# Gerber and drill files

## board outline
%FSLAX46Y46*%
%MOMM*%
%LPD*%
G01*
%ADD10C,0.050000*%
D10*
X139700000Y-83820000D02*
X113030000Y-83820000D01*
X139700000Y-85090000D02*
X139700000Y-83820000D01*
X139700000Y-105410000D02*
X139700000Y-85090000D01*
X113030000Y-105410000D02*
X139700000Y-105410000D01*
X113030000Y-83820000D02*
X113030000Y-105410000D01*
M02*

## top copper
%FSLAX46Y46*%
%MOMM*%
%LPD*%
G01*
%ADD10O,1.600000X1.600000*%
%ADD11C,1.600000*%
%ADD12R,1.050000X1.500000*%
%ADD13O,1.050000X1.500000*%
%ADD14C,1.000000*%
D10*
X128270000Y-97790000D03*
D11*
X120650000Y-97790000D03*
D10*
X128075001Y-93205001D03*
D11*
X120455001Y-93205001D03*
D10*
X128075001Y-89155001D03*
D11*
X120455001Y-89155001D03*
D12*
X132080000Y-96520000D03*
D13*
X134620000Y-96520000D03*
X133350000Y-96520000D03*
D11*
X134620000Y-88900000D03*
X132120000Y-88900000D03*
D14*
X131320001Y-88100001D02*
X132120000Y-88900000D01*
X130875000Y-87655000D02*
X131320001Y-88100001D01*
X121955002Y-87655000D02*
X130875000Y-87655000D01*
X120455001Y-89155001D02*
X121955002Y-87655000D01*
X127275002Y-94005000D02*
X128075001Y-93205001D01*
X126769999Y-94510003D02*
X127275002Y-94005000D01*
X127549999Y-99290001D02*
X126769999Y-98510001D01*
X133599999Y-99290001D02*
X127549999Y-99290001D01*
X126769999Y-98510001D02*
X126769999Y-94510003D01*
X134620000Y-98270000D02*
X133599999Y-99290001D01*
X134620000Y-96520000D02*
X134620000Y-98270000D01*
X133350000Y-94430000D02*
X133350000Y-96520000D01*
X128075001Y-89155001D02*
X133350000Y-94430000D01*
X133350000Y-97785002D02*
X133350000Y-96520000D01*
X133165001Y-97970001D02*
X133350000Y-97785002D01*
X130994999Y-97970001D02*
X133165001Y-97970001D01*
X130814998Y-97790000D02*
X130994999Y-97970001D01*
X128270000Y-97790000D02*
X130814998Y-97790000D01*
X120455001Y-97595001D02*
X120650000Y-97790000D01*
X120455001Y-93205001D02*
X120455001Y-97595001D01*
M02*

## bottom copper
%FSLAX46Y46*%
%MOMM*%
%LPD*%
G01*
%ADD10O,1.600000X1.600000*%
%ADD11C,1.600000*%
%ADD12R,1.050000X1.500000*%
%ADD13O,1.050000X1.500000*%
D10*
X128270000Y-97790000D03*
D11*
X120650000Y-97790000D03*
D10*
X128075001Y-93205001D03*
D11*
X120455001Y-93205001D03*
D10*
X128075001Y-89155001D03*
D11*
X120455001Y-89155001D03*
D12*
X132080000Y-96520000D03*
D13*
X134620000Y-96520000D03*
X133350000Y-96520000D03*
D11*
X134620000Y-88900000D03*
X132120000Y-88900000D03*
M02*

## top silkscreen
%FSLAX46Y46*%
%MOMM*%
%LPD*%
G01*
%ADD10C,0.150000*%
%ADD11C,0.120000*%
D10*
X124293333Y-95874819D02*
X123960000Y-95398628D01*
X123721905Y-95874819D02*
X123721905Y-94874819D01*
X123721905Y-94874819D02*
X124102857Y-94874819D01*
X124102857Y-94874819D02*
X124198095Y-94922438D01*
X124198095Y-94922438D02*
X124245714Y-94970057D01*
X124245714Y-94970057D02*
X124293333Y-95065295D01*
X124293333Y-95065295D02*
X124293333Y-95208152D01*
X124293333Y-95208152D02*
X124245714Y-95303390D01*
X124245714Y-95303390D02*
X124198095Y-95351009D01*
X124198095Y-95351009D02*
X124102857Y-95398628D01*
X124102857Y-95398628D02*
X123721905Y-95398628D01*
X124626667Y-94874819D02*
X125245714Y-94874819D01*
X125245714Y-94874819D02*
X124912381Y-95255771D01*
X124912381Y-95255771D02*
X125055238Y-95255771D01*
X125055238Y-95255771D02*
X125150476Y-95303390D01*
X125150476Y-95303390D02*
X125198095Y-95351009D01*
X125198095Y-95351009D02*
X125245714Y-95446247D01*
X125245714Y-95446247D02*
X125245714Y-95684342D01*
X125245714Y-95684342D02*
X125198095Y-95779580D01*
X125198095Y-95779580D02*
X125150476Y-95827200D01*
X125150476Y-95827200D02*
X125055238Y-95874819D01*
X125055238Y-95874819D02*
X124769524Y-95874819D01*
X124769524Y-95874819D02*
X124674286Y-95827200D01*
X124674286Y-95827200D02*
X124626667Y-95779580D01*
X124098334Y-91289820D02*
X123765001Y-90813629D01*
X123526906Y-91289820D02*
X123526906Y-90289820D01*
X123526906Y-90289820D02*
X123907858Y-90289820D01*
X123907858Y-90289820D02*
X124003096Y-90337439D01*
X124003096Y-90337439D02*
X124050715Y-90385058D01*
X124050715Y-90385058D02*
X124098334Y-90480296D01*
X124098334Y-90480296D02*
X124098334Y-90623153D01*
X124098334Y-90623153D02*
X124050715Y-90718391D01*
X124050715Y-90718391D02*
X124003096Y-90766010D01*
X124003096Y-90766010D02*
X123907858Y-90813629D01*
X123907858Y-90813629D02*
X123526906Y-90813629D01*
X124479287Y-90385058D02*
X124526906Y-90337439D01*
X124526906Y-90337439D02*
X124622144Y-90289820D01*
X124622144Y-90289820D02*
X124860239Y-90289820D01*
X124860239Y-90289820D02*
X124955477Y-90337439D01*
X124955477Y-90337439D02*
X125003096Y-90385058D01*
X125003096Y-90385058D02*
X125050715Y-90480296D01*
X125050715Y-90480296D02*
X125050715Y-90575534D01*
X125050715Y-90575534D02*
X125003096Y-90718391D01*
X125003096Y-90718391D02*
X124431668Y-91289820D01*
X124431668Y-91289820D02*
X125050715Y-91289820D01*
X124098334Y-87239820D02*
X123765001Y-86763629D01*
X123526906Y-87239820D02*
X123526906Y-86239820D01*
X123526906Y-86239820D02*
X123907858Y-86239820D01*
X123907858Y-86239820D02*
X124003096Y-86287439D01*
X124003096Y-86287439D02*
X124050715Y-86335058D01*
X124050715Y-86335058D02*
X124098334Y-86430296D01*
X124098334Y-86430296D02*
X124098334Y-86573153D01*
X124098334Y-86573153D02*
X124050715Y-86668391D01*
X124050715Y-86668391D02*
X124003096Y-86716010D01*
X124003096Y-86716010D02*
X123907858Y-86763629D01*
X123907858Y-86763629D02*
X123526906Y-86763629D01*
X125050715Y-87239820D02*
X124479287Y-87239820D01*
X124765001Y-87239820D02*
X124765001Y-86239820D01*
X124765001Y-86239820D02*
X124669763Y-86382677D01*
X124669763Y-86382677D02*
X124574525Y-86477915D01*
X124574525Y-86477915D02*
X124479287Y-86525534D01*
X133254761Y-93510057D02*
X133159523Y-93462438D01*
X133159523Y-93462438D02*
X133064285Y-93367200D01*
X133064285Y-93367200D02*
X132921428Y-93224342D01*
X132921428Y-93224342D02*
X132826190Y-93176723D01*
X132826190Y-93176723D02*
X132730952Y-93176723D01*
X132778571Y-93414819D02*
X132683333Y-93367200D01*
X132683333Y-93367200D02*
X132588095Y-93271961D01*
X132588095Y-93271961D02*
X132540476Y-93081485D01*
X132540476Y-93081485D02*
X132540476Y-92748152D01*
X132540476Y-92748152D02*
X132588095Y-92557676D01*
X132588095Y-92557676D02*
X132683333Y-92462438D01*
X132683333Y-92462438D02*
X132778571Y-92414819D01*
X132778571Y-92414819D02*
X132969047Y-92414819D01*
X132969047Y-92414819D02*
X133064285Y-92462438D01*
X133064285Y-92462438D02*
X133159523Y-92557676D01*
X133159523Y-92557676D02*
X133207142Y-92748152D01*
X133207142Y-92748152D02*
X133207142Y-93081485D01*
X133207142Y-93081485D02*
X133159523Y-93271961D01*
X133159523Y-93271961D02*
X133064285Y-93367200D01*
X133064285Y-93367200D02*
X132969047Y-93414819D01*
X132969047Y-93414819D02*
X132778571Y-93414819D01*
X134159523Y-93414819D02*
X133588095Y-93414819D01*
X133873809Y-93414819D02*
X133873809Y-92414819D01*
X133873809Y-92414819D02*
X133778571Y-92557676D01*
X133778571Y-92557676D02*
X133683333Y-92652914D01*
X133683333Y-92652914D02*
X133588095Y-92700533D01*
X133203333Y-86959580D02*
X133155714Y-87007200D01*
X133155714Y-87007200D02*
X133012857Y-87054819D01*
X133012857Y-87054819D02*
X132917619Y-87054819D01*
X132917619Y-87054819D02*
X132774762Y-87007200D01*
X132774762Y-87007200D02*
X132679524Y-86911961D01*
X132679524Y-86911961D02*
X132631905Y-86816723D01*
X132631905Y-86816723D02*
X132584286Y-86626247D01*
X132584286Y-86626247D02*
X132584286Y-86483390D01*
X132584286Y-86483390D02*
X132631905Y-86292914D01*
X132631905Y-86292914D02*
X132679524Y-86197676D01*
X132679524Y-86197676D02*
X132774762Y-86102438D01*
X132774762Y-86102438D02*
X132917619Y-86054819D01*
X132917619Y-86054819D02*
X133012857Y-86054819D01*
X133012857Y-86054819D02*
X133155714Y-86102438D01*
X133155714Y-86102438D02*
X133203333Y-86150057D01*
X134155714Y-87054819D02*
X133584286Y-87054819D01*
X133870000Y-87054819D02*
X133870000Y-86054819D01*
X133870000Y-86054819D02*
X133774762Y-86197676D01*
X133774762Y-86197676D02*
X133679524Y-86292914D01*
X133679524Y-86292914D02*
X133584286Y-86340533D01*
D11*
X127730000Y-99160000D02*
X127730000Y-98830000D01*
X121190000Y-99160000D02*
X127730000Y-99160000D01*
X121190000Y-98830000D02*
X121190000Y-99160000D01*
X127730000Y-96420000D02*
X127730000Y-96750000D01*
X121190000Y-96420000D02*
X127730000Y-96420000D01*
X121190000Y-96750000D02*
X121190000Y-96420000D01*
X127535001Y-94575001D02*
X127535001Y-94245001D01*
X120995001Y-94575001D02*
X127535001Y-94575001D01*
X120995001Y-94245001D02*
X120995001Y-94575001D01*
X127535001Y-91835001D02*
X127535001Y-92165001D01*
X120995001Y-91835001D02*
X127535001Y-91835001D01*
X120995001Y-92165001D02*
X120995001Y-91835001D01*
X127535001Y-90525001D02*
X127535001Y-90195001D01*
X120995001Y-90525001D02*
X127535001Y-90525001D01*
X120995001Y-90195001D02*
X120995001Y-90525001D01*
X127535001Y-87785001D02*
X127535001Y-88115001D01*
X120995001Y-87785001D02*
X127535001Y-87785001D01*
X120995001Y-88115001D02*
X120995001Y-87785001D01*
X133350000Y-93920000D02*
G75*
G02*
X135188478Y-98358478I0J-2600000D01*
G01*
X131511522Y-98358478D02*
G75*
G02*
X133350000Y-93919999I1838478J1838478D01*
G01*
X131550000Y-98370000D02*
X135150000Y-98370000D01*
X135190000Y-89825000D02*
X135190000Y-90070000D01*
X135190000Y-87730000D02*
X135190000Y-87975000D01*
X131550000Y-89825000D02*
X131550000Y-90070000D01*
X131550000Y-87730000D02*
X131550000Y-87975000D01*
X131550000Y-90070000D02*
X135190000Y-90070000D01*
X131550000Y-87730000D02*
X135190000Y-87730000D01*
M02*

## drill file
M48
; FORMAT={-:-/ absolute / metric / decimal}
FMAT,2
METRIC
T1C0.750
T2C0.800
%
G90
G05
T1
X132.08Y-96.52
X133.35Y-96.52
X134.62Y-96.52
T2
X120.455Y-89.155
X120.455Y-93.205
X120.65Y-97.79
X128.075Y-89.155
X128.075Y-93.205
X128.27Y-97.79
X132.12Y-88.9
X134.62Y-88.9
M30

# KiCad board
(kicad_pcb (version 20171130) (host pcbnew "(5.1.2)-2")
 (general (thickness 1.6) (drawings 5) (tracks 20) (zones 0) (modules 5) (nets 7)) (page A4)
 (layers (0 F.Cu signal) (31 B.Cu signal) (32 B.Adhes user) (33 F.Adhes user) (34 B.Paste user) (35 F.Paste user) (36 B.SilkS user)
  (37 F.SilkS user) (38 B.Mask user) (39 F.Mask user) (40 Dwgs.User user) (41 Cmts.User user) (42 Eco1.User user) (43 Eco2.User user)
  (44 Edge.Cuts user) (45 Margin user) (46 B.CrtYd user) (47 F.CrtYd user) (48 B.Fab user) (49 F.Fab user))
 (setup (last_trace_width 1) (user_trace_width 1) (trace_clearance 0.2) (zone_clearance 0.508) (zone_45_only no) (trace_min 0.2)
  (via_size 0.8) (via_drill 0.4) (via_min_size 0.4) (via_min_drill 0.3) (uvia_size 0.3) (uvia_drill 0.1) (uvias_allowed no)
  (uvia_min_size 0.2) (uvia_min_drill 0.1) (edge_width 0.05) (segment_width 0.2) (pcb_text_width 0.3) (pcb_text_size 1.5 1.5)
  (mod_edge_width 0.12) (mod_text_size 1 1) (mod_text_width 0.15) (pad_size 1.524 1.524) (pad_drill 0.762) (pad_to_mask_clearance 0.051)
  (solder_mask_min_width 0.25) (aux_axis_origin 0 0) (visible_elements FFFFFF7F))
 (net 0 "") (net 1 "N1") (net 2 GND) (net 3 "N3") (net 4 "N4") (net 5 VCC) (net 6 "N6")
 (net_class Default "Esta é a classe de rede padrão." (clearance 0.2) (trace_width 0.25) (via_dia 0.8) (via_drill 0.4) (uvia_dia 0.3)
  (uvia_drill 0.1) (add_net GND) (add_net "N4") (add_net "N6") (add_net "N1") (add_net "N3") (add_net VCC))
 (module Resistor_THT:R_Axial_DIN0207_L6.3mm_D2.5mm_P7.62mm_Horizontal (layer F.Cu) (at 120.65 97.79)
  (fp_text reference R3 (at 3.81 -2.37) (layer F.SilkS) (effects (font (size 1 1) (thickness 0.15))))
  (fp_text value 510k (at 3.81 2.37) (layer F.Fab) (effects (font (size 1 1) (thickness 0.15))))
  (fp_line (start 7.08 1.37) (end 7.08 1.04) (layer F.SilkS) (width 0.12))
  (fp_line (start 0.54 1.37) (end 7.08 1.37) (layer F.SilkS) (width 0.12))
  (fp_line (start 0.54 1.04) (end 0.54 1.37) (layer F.SilkS) (width 0.12))
  (fp_line (start 7.08 -1.37) (end 7.08 -1.04) (layer F.SilkS) (width 0.12))
  (fp_line (start 0.54 -1.37) (end 7.08 -1.37) (layer F.SilkS) (width 0.12))
  (fp_line (start 0.54 -1.04) (end 0.54 -1.37) (layer F.SilkS) (width 0.12))
  (pad 2 thru_hole oval (at 7.62 0) (size 1.6 1.6) (drill 0.8) (layers *.Cu *.Mask) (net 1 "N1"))
  (pad 1 thru_hole circle (at 0 0) (size 1.6 1.6) (drill 0.8) (layers *.Cu *.Mask) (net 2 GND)))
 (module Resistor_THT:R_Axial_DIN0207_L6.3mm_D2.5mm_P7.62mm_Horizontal (layer F.Cu) (at 120.455001 93.205001)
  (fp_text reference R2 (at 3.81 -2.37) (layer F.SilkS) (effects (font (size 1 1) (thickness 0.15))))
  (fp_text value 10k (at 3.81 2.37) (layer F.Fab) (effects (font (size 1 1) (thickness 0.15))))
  (fp_line (start 7.08 1.37) (end 7.08 1.04) (layer F.SilkS) (width 0.12))
  (fp_line (start 0.54 1.37) (end 7.08 1.37) (layer F.SilkS) (width 0.12))
  (fp_line (start 0.54 1.04) (end 0.54 1.37) (layer F.SilkS) (width 0.12))
  (fp_line (start 7.08 -1.37) (end 7.08 -1.04) (layer F.SilkS) (width 0.12))
  (fp_line (start 0.54 -1.37) (end 7.08 -1.37) (layer F.SilkS) (width 0.12))
  (fp_line (start 0.54 -1.04) (end 0.54 -1.37) (layer F.SilkS) (width 0.12))
  (pad 2 thru_hole oval (at 7.62 0) (size 1.6 1.6) (drill 0.8) (layers *.Cu *.Mask) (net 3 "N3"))
  (pad 1 thru_hole circle (at 0 0) (size 1.6 1.6) (drill 0.8) (layers *.Cu *.Mask) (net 2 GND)))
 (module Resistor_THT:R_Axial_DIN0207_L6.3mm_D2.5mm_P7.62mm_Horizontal (layer F.Cu) (at 120.455001 89.155001)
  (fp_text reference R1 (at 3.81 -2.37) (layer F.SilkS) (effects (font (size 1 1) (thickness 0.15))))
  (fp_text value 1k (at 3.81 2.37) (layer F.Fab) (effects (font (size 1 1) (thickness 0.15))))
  (fp_line (start 7.08 1.37) (end 7.08 1.04) (layer F.SilkS) (width 0.12))
  (fp_line (start 0.54 1.37) (end 7.08 1.37) (layer F.SilkS) (width 0.12))
  (fp_line (start 0.54 1.04) (end 0.54 1.37) (layer F.SilkS) (width 0.12))
  (fp_line (start 7.08 -1.37) (end 7.08 -1.04) (layer F.SilkS) (width 0.12))
  (fp_line (start 0.54 -1.37) (end 7.08 -1.37) (layer F.SilkS) (width 0.12))
  (fp_line (start 0.54 -1.04) (end 0.54 -1.37) (layer F.SilkS) (width 0.12))
  (pad 2 thru_hole oval (at 7.62 0) (size 1.6 1.6) (drill 0.8) (layers *.Cu *.Mask) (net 1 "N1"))
  (pad 1 thru_hole circle (at 0 0) (size 1.6 1.6) (drill 0.8) (layers *.Cu *.Mask) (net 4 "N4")))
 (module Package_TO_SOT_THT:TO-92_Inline (layer F.Cu) (at 132.08 96.52)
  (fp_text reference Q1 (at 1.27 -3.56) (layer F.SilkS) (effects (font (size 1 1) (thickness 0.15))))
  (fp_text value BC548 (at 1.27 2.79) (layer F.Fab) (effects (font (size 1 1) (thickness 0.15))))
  (fp_arc (start 1.27 0) (end 1.27 -2.6) (angle 135) (layer F.SilkS) (width 0.12))
  (fp_arc (start 1.27 0) (end 1.27 -2.6) (angle -135) (layer F.SilkS) (width 0.12))
  (fp_line (start -0.53 1.85) (end 3.07 1.85) (layer F.SilkS) (width 0.12))
  (pad 1 thru_hole rect (at 0 0) (size 1.05 1.5) (drill 0.75) (layers *.Cu *.Mask) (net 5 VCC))
  (pad 3 thru_hole oval (at 2.54 0) (size 1.05 1.5) (drill 0.75) (layers *.Cu *.Mask) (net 3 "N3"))
  (pad 2 thru_hole oval (at 1.27 0) (size 1.05 1.5) (drill 0.75) (layers *.Cu *.Mask) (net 1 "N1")))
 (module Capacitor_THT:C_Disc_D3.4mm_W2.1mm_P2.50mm (layer F.Cu) (at 132.12 88.9)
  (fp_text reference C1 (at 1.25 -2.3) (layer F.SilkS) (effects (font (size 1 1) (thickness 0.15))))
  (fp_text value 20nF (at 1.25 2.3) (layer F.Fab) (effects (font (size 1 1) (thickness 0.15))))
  (fp_line (start 3.07 0.925) (end 3.07 1.17) (layer F.SilkS) (width 0.12))
  (fp_line (start 3.07 -1.17) (end 3.07 -0.925) (layer F.SilkS) (width 0.12))
  (fp_line (start -0.57 0.925) (end -0.57 1.17) (layer F.SilkS) (width 0.12))
  (fp_line (start -0.57 -1.17) (end -0.57 -0.925) (layer F.SilkS) (width 0.12))
  (fp_line (start -0.57 1.17) (end 3.07 1.17) (layer F.SilkS) (width 0.12))
  (fp_line (start -0.57 -1.17) (end 3.07 -1.17) (layer F.SilkS) (width 0.12))
  (pad 2 thru_hole circle (at 2.5 0) (size 1.6 1.6) (drill 0.8) (layers *.Cu *.Mask) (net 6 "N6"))
  (pad 1 thru_hole circle (at 0 0) (size 1.6 1.6) (drill 0.8) (layers *.Cu *.Mask) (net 4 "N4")))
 (gr_line (start 139.7 83.82) (end 113.03 83.82) (layer Edge.Cuts) (width 0.05))
 (gr_line (start 139.7 85.09) (end 139.7 83.82) (layer Edge.Cuts) (width 0.05))
 (gr_line (start 139.7 105.41) (end 139.7 85.09) (layer Edge.Cuts) (width 0.05))
 (gr_line (start 113.03 105.41) (end 139.7 105.41) (layer Edge.Cuts) (width 0.05))
 (gr_line (start 113.03 83.82) (end 113.03 105.41) (layer Edge.Cuts) (width 0.05))
 (segment (start 131.320001 88.100001) (end 132.12 88.9) (width 1) (layer F.Cu) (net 4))
 (segment (start 130.875 87.655) (end 131.320001 88.100001) (width 1) (layer F.Cu) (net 4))
 (segment (start 121.955002 87.655) (end 130.875 87.655) (width 1) (layer F.Cu) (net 4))
 (segment (start 120.455001 89.155001) (end 121.955002 87.655) (width 1) (layer F.Cu) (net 4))
 (segment (start 127.275002 94.005) (end 128.075001 93.205001) (width 1) (layer F.Cu) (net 3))
 (segment (start 126.769999 94.510003) (end 127.275002 94.005) (width 1) (layer F.Cu) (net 3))
 (segment (start 127.549999 99.290001) (end 126.769999 98.510001) (width 1) (layer F.Cu) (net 3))
 (segment (start 133.599999 99.290001) (end 127.549999 99.290001) (width 1) (layer F.Cu) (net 3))
 (segment (start 126.769999 98.510001) (end 126.769999 94.510003) (width 1) (layer F.Cu) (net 3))
 (segment (start 134.62 98.27) (end 133.599999 99.290001) (width 1) (layer F.Cu) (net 3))
 (segment (start 134.62 96.52) (end 134.62 98.27) (width 1) (layer F.Cu) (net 3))
 (segment (start 133.35 94.43) (end 133.35 96.52) (width 1) (layer F.Cu) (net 1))
 (segment (start 128.075001 89.155001) (end 133.35 94.43) (width 1) (layer F.Cu) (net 1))
 (segment (start 133.35 97.785002) (end 133.35 96.52) (width 1) (layer F.Cu) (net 1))
 (segment (start 133.165001 97.970001) (end 133.35 97.785002) (width 1) (layer F.Cu) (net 1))
 (segment (start 130.994999 97.970001) (end 133.165001 97.970001) (width 1) (layer F.Cu) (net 1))
 (segment (start 130.814998 97.79) (end 130.994999 97.970001) (width 1) (layer F.Cu) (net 1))
 (segment (start 128.27 97.79) (end 130.814998 97.79) (width 1) (layer F.Cu) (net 1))
 (segment (start 120.455001 97.595001) (end 120.65 97.79) (width 1) (layer F.Cu) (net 2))
 (segment (start 120.455001 93.205001) (end 120.455001 97.595001) (width 1) (layer F.Cu) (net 2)))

